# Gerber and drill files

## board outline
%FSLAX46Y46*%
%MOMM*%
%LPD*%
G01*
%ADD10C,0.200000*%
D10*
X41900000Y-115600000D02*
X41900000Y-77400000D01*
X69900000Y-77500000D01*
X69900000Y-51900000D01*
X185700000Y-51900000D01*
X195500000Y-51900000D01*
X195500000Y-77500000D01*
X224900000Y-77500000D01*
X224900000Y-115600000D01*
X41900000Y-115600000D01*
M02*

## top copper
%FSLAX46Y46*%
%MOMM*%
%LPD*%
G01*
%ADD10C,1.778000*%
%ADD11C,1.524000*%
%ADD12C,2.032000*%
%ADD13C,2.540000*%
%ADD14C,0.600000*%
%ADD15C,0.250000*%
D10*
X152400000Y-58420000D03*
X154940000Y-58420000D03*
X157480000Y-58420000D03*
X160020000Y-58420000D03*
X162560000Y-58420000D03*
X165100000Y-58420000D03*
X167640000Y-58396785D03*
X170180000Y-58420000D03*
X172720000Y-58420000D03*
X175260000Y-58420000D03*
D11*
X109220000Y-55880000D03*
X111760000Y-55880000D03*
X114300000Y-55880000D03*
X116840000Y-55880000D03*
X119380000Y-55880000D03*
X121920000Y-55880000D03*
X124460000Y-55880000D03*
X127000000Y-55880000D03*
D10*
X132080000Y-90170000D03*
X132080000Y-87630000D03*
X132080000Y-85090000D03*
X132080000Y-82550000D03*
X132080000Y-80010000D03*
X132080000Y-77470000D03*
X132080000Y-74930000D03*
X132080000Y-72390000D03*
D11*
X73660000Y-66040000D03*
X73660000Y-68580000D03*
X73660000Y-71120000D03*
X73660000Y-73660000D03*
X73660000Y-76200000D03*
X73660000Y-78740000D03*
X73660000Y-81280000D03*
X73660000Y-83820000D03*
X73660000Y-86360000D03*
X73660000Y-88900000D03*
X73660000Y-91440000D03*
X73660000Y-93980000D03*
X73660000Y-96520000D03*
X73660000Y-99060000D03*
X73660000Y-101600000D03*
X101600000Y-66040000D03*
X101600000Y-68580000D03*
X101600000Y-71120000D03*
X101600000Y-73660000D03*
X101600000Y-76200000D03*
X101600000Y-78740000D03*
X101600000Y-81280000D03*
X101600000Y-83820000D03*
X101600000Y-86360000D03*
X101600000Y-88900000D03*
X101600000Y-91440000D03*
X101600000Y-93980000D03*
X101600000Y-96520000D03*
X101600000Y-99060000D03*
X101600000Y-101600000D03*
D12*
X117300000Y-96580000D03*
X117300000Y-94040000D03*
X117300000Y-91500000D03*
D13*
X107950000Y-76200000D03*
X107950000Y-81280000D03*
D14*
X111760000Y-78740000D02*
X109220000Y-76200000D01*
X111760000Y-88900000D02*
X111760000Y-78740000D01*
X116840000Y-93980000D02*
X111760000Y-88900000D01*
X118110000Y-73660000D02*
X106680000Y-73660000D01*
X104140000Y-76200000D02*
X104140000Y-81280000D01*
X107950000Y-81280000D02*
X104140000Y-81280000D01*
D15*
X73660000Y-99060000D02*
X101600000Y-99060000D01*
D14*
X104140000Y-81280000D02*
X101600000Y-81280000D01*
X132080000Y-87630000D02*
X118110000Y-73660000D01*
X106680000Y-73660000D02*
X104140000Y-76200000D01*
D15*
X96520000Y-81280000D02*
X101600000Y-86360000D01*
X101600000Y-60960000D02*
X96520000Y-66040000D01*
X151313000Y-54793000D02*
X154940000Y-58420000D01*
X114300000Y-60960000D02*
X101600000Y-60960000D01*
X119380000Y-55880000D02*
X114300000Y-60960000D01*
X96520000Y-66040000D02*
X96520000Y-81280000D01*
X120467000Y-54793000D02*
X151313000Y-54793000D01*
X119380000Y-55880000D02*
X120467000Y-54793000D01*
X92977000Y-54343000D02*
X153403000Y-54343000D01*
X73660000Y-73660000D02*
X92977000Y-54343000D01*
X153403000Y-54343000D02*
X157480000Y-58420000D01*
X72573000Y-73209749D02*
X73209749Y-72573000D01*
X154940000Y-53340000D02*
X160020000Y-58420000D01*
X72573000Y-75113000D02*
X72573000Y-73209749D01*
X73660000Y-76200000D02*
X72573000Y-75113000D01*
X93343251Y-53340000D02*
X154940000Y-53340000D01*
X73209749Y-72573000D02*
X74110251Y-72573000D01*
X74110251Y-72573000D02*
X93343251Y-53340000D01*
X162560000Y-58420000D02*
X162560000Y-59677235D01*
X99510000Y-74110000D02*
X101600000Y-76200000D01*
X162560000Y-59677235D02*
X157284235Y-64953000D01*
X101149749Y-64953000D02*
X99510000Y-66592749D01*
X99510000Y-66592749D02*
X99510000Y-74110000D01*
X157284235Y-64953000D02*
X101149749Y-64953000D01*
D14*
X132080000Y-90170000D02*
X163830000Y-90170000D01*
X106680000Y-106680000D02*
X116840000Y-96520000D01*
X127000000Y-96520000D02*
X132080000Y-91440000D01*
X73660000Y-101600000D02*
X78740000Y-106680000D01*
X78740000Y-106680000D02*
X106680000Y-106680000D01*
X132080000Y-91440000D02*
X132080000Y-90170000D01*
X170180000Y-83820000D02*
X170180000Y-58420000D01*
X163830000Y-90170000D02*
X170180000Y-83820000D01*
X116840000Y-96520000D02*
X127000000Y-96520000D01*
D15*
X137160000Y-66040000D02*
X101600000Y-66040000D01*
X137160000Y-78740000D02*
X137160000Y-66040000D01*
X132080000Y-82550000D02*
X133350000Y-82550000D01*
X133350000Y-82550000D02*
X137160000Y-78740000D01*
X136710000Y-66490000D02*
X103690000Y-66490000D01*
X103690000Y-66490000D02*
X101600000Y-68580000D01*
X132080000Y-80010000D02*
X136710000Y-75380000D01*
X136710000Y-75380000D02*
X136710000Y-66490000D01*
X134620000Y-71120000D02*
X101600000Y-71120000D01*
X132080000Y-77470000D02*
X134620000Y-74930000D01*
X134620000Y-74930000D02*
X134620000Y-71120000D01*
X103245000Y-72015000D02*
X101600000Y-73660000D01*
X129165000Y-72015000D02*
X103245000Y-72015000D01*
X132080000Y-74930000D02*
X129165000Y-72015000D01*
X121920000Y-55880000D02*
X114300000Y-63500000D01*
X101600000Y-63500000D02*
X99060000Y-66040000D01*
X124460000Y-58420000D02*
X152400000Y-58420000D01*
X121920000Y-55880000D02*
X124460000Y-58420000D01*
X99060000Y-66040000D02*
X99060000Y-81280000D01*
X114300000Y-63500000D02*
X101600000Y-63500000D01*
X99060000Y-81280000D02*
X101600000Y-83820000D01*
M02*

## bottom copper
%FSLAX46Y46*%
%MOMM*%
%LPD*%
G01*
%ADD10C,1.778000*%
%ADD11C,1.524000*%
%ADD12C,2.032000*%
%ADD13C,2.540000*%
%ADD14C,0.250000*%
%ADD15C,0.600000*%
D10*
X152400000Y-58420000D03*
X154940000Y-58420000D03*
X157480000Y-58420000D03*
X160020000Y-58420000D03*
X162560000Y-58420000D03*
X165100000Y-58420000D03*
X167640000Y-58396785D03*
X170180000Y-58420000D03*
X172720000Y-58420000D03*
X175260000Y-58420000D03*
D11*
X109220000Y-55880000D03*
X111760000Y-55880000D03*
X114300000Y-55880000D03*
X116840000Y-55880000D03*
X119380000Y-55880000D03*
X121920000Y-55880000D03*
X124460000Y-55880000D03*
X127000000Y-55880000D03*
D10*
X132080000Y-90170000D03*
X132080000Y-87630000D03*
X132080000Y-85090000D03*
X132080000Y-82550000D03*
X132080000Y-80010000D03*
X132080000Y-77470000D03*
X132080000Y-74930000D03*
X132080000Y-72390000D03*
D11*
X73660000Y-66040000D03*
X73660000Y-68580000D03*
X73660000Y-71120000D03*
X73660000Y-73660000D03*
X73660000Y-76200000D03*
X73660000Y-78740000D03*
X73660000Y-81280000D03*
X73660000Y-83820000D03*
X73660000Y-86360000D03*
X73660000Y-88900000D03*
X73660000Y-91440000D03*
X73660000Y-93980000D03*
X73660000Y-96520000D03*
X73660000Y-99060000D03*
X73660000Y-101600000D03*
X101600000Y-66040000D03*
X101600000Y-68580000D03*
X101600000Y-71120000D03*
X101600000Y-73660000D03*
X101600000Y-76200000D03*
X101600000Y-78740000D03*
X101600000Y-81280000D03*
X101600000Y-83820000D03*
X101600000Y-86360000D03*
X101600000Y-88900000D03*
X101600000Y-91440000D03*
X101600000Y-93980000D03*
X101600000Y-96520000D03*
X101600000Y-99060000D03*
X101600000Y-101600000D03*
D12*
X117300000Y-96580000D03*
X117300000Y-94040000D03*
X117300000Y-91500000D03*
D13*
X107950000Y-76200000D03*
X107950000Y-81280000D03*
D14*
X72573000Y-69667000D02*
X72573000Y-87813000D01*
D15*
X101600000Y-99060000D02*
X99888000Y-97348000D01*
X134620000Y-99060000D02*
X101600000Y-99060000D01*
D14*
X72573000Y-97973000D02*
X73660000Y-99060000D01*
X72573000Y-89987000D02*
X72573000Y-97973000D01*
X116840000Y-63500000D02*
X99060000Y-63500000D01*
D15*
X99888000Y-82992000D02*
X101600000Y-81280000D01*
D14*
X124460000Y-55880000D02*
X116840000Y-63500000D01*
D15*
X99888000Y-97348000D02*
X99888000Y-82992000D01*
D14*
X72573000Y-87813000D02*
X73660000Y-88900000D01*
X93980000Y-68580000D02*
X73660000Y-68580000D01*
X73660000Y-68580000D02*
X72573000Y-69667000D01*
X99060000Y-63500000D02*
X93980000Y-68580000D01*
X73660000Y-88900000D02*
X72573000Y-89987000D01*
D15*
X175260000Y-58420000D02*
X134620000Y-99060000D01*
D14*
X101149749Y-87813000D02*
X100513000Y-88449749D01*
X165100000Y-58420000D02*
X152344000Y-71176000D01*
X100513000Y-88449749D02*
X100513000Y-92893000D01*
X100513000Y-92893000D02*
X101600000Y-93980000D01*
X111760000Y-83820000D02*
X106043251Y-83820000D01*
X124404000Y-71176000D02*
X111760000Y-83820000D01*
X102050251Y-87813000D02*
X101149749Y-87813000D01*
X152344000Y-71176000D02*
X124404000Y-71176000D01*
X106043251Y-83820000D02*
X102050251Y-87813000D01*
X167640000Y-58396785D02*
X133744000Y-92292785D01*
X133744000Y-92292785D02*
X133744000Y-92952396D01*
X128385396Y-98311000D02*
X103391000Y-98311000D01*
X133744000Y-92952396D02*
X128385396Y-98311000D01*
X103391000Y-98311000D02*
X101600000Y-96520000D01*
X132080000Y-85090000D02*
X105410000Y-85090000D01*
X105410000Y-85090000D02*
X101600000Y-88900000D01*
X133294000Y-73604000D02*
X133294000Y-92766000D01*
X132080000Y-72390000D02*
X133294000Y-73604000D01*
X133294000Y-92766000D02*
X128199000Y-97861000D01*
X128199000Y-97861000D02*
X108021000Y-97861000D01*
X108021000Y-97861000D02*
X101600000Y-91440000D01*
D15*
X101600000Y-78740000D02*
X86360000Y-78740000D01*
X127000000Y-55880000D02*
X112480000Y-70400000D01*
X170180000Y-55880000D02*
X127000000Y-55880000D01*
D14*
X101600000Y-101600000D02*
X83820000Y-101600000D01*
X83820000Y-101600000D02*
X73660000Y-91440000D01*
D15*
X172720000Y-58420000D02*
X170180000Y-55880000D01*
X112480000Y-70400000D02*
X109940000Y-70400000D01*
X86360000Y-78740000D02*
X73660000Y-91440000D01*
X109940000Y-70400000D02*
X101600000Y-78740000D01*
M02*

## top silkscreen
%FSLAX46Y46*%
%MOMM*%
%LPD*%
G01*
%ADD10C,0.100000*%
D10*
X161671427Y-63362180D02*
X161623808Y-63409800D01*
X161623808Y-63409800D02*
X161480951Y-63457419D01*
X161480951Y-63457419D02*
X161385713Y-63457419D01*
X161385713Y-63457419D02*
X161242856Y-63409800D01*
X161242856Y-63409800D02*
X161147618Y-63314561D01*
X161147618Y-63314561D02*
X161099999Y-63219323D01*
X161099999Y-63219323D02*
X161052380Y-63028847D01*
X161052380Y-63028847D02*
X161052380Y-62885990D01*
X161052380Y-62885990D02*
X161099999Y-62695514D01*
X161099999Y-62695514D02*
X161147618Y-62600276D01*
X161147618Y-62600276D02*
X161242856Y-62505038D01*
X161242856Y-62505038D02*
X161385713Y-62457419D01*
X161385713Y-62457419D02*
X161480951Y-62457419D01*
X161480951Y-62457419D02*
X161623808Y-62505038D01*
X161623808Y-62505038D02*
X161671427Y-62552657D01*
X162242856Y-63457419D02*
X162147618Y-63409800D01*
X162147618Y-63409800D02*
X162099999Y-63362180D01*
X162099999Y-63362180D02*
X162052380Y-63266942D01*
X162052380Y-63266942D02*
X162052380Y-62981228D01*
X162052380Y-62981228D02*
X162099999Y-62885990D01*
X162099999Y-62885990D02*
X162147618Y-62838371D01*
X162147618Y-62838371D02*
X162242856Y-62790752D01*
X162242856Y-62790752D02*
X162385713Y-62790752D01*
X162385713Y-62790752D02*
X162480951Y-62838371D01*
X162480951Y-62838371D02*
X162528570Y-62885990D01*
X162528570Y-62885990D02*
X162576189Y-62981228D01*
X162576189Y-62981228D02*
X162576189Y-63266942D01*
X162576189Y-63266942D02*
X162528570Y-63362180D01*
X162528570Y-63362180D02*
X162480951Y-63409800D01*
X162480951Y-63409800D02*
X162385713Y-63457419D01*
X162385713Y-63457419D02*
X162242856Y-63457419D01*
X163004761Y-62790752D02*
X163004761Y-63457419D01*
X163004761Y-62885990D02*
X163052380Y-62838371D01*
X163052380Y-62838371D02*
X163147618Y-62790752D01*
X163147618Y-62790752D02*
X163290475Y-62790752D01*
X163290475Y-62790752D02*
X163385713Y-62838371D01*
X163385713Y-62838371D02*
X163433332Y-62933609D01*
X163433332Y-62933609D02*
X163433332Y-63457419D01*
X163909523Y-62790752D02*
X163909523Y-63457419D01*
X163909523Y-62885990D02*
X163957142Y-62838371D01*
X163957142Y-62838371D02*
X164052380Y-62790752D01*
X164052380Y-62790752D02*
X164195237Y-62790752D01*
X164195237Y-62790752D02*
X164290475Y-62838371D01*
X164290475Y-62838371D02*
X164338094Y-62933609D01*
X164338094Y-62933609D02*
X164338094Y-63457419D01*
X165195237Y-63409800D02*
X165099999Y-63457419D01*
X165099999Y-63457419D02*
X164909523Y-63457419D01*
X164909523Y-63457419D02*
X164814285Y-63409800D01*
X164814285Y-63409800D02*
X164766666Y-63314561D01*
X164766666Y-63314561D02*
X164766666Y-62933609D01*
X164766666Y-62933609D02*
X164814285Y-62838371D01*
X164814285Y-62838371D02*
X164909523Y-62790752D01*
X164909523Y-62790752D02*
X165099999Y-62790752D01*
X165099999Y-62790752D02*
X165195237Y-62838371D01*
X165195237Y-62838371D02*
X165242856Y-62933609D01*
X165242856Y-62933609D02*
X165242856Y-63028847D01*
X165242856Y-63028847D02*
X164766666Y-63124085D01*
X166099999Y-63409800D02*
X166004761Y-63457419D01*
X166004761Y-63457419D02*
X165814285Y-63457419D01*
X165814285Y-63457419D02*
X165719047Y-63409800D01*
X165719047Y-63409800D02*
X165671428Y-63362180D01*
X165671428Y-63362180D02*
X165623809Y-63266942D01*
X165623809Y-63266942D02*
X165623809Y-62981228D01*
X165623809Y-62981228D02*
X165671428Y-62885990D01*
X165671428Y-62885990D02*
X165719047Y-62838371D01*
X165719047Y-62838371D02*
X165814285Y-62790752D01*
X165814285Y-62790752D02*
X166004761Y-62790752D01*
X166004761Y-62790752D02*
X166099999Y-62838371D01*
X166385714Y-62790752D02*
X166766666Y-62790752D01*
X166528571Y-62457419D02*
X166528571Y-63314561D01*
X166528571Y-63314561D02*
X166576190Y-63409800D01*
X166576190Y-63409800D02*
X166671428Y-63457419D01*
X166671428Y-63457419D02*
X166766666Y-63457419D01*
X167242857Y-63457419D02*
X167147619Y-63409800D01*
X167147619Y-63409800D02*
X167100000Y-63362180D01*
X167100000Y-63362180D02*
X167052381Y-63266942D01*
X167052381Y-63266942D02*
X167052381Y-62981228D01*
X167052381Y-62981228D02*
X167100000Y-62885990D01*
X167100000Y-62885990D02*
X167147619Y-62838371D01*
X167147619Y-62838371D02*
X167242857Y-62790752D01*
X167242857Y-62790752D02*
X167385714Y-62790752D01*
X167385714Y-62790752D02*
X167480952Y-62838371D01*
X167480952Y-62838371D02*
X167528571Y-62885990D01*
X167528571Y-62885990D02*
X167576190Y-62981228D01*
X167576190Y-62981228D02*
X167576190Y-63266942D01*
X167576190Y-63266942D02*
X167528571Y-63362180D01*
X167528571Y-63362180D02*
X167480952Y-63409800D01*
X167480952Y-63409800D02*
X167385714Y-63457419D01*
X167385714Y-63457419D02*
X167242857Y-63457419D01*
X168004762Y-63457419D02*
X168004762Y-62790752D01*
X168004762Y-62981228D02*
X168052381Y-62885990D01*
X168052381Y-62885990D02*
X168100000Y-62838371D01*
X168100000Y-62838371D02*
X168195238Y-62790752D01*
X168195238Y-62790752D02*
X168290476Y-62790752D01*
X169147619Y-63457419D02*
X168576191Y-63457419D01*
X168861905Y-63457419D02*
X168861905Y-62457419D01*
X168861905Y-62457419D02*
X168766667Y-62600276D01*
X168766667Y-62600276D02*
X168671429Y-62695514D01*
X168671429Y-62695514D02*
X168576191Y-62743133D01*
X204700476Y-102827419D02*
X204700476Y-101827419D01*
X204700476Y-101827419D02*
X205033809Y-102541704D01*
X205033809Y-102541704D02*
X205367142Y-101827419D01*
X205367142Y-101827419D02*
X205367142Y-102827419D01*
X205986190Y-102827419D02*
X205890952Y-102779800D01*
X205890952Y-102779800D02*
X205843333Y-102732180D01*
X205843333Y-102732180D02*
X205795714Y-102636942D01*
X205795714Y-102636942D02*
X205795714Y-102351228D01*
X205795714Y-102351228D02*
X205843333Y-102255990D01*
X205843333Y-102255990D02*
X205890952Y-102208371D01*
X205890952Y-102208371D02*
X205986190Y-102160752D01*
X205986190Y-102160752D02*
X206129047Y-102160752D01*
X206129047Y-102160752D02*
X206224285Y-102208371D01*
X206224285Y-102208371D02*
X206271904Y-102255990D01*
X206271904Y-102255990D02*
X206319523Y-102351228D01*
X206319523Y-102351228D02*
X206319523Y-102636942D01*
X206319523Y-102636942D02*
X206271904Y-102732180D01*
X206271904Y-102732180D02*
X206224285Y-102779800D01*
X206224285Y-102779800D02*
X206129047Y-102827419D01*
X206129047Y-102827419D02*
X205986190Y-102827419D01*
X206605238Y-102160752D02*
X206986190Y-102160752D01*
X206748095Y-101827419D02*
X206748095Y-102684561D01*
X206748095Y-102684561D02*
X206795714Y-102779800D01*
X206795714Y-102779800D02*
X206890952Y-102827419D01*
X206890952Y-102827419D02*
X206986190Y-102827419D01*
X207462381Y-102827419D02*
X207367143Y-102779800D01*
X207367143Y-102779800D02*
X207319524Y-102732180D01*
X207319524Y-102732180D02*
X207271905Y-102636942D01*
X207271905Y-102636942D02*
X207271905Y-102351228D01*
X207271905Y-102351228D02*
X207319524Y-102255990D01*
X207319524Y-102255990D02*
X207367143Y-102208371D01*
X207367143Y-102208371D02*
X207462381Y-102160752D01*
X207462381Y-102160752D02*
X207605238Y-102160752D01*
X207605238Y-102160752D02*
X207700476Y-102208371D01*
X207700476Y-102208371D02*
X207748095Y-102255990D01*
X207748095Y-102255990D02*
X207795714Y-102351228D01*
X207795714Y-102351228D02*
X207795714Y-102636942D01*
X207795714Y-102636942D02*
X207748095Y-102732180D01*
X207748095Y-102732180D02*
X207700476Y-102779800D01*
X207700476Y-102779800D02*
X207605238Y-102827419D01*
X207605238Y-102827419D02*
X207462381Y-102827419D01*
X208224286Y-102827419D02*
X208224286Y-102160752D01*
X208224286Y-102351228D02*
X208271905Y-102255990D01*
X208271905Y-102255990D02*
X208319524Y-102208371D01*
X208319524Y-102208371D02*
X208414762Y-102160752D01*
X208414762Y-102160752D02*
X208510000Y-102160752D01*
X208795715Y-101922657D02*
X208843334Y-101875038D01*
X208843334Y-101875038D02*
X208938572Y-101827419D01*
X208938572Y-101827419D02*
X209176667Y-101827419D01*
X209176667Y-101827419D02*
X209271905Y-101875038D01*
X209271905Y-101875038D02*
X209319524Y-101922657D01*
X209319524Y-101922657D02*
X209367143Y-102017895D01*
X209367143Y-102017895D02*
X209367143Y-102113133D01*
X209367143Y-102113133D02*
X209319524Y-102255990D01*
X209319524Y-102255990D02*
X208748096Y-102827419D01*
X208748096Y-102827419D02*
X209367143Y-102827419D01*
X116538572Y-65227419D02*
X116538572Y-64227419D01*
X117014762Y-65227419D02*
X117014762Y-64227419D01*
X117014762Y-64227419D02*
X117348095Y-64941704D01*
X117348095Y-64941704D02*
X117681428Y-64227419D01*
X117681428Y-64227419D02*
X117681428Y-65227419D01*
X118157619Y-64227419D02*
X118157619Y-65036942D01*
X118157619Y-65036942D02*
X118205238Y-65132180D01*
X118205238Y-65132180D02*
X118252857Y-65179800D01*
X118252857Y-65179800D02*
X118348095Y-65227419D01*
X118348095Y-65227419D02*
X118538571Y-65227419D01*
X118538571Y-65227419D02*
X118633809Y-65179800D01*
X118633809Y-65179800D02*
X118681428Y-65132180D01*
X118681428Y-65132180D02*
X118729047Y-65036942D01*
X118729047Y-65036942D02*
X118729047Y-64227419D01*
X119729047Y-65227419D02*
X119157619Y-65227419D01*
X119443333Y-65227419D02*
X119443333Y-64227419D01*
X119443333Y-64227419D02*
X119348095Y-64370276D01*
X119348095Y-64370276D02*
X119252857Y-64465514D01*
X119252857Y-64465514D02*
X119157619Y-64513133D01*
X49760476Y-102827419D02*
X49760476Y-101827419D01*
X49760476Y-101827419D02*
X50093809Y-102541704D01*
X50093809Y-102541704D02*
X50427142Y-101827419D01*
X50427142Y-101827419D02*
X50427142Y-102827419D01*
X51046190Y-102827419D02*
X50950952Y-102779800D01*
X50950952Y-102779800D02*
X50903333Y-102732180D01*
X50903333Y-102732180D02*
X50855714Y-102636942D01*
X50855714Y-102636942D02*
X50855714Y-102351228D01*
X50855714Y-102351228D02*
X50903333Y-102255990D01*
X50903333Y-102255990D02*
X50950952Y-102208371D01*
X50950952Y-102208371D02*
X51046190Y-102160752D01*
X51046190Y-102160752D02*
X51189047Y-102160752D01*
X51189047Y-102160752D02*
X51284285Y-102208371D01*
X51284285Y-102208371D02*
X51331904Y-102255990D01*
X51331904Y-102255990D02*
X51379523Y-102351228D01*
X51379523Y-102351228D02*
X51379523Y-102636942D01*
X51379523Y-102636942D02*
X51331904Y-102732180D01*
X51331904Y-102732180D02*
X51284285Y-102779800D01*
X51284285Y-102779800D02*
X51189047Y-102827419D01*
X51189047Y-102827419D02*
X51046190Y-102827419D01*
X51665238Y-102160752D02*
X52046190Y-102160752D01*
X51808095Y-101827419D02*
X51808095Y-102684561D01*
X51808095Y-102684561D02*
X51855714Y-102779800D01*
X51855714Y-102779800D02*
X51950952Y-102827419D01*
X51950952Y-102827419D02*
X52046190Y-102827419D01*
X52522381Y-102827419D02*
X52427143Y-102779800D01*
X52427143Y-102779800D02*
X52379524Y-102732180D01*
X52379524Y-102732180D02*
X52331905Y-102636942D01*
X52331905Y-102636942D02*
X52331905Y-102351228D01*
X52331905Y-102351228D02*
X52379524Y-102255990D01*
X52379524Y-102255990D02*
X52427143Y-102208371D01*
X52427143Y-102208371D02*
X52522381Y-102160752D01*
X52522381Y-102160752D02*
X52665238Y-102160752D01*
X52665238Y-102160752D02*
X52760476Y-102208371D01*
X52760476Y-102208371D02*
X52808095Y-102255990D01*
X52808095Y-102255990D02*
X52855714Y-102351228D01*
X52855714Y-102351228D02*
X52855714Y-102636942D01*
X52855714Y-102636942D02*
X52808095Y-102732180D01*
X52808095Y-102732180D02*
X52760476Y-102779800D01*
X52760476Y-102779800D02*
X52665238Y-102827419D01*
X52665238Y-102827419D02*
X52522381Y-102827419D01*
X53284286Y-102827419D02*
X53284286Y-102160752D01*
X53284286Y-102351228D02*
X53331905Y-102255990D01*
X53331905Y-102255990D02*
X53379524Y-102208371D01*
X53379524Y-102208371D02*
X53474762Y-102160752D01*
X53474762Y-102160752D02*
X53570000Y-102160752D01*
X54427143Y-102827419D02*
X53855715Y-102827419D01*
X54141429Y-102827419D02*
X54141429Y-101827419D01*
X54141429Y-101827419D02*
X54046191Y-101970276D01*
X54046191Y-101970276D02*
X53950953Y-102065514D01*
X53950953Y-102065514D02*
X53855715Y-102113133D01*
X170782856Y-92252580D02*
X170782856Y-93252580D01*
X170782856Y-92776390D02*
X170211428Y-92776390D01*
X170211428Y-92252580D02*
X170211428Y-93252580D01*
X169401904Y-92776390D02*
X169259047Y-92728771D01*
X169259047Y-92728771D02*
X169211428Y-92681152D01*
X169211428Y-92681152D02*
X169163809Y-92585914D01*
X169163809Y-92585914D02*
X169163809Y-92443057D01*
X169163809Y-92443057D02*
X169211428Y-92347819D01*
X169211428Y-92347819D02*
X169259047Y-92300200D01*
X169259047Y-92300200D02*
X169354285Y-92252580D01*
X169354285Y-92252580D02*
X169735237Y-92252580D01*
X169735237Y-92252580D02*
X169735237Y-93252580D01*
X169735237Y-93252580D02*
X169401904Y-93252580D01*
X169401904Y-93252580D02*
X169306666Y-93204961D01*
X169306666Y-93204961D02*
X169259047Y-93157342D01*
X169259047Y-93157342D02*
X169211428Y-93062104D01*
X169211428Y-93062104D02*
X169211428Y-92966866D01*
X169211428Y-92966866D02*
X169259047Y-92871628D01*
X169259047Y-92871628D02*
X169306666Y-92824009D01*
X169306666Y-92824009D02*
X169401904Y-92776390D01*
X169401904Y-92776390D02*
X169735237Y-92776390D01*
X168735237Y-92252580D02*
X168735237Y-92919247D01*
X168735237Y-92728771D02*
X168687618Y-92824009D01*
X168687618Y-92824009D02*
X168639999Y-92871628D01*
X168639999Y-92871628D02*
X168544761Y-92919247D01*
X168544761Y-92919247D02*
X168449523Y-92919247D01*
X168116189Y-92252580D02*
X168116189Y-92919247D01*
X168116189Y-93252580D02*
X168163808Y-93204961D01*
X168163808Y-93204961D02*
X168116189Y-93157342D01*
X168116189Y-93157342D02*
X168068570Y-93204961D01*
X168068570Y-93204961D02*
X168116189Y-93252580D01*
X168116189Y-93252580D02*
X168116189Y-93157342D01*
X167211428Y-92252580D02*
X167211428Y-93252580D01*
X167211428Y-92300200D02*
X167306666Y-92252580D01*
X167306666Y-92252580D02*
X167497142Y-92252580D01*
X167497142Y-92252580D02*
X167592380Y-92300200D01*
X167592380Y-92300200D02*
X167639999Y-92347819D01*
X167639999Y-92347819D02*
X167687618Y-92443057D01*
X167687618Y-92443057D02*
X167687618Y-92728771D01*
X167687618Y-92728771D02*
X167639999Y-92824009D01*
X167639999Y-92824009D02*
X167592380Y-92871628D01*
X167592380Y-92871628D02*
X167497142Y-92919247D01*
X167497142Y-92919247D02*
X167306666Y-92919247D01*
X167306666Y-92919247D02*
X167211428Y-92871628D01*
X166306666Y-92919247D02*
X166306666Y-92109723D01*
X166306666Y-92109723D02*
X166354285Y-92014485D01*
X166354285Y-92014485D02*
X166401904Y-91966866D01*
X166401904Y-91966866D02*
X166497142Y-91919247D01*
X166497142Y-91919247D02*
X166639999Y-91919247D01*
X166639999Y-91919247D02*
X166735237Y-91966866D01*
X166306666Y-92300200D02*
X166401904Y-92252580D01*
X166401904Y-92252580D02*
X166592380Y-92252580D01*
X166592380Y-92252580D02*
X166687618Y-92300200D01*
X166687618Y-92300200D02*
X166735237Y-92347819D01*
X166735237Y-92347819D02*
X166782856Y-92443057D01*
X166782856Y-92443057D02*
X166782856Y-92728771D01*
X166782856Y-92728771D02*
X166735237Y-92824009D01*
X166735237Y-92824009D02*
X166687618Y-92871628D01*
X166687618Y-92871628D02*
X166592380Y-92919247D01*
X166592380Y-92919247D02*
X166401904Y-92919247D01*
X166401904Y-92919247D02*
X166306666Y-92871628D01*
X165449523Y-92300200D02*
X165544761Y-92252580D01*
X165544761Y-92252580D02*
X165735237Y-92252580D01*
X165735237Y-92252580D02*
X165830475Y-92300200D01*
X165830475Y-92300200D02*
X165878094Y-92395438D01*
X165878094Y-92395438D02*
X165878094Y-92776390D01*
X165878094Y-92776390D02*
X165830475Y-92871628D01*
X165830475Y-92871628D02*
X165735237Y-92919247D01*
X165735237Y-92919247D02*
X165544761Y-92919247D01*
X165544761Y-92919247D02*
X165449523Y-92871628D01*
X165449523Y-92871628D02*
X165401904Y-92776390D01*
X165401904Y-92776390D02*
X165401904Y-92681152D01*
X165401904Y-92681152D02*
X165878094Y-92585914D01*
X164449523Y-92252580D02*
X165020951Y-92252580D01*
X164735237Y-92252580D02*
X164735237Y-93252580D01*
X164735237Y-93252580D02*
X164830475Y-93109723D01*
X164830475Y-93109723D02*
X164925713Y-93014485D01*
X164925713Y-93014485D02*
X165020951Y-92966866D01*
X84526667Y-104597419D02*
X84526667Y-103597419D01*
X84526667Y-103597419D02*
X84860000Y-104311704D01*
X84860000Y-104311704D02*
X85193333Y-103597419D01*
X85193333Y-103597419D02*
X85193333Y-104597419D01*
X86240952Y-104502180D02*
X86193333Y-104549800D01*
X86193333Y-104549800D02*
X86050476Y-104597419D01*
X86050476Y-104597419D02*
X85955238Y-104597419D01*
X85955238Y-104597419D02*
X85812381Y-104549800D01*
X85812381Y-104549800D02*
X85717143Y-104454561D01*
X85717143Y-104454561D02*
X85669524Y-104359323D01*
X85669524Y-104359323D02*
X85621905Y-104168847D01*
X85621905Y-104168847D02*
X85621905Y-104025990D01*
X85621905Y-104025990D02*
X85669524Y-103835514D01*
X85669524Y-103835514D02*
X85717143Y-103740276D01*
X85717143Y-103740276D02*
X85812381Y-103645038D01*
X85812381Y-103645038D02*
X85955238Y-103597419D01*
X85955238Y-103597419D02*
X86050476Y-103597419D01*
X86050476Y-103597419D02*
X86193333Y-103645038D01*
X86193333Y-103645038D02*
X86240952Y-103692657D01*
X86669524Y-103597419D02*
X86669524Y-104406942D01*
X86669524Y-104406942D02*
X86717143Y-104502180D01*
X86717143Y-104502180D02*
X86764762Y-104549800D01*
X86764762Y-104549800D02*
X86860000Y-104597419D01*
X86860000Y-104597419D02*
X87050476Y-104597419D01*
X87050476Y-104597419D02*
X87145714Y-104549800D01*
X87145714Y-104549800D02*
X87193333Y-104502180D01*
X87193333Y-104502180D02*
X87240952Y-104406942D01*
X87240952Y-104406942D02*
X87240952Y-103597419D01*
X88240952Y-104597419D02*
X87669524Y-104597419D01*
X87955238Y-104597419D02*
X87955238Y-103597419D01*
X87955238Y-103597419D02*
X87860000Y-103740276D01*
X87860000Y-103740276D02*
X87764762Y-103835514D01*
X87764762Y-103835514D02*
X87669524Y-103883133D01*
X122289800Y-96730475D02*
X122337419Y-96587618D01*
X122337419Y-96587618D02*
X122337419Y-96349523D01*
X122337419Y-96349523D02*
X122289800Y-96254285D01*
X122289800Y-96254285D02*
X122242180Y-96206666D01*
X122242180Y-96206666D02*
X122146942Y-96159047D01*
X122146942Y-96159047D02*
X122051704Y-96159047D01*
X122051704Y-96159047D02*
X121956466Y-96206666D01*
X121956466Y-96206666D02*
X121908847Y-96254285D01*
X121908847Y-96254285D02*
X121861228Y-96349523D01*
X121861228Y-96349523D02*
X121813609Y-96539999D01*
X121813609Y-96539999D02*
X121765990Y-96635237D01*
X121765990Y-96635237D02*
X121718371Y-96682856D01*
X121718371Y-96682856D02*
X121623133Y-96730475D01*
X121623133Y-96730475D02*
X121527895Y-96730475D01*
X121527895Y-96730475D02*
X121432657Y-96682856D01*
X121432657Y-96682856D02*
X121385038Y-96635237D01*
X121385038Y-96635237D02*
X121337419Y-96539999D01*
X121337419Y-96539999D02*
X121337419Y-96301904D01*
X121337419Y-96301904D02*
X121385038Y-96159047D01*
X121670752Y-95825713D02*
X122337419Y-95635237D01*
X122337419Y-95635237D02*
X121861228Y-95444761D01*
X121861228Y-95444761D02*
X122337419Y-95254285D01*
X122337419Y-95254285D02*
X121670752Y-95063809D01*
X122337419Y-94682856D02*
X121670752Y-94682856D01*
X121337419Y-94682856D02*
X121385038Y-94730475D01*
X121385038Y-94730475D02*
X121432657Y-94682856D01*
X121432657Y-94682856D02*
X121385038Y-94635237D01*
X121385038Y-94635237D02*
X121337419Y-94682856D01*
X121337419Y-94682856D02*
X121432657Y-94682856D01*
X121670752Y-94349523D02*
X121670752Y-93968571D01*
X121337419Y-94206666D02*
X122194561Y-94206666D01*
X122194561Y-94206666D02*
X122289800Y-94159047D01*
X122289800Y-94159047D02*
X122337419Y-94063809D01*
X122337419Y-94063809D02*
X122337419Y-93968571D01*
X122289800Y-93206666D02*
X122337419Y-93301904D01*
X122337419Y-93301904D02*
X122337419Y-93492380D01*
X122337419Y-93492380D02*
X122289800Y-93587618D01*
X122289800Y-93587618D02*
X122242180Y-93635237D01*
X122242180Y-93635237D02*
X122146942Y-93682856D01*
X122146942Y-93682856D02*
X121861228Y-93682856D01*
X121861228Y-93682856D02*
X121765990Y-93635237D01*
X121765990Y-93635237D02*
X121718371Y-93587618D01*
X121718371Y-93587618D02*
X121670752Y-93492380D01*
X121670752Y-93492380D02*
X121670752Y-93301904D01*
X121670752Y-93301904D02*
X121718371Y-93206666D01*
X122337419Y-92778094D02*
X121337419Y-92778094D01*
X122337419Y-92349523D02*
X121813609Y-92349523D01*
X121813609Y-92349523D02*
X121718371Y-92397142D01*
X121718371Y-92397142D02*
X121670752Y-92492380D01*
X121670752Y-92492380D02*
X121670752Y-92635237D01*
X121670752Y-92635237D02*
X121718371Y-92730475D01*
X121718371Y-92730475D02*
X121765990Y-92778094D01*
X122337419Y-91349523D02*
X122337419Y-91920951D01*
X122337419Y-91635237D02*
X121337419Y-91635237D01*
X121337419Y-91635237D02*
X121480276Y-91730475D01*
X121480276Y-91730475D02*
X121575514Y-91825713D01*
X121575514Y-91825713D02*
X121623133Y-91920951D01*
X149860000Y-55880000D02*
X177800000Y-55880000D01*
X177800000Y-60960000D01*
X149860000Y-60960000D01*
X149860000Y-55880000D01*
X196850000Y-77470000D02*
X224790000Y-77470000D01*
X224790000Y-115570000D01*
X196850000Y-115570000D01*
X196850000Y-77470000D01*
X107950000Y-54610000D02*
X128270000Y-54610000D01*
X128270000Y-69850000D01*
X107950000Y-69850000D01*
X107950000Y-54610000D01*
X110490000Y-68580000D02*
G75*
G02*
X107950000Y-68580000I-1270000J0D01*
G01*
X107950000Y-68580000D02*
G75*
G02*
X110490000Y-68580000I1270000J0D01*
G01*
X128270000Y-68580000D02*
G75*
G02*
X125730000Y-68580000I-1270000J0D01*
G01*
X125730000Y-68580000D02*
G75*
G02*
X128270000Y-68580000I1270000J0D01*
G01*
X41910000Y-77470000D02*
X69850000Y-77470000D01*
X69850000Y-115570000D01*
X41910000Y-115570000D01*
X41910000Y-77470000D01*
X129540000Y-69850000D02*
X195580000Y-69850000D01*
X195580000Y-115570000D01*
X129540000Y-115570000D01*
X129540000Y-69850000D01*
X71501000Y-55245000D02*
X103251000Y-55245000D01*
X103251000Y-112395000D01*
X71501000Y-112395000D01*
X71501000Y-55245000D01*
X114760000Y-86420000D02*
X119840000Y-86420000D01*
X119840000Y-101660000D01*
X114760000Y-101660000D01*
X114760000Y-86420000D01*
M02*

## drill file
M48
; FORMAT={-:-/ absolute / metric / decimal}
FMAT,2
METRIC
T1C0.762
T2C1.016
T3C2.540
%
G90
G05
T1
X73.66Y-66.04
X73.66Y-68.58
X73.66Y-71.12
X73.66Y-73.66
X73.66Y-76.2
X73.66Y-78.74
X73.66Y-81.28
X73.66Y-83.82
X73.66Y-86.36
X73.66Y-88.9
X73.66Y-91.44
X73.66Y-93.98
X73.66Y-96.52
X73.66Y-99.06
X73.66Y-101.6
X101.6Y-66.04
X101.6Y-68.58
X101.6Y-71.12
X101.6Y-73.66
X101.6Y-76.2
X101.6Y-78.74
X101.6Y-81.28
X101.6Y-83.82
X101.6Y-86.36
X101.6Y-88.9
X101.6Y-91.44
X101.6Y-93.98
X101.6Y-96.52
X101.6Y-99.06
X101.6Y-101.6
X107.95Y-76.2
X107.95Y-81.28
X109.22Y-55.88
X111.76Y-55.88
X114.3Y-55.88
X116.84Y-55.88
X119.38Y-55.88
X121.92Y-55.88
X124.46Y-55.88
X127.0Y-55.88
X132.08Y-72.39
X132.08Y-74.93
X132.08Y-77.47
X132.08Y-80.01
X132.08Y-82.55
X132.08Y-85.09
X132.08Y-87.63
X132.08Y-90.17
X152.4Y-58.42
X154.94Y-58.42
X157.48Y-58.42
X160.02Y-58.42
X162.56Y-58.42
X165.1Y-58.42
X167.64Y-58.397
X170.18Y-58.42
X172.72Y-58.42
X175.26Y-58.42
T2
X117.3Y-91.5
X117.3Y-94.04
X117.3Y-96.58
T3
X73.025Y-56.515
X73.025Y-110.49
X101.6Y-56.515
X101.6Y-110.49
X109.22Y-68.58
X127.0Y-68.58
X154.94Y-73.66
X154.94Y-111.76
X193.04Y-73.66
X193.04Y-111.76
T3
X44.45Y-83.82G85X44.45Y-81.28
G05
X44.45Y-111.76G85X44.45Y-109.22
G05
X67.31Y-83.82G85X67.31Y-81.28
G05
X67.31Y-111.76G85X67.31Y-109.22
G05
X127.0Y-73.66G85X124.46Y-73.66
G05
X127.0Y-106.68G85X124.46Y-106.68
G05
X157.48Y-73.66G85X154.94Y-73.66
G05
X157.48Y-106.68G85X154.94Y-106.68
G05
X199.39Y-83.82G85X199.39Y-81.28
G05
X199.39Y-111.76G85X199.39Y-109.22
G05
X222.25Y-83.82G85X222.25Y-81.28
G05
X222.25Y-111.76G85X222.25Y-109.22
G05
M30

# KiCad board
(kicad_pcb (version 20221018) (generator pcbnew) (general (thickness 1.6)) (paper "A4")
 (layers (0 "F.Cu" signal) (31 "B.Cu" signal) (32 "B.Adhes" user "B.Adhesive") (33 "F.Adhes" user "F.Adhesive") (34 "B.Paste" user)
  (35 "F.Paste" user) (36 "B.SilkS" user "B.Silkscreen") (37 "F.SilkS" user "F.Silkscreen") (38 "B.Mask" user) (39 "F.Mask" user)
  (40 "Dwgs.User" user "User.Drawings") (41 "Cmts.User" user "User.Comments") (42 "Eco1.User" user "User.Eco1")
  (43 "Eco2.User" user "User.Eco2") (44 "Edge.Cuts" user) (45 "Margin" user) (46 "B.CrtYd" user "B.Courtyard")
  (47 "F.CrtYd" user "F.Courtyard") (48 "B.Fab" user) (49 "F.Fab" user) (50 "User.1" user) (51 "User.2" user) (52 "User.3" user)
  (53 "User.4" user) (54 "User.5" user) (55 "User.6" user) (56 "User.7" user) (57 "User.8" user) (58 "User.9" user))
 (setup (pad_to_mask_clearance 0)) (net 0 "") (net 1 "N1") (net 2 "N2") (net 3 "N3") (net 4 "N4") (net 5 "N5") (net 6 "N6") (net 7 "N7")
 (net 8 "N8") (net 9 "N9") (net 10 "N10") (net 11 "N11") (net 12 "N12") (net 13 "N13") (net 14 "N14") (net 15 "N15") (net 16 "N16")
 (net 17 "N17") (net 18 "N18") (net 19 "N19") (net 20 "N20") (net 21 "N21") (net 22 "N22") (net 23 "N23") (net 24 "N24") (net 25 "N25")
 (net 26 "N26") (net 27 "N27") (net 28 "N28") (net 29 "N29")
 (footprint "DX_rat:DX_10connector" (layer "F.Cu") (at 165.1 63.5)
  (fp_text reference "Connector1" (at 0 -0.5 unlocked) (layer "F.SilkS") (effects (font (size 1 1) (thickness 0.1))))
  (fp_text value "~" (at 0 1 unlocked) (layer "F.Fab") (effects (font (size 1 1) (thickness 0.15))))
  (fp_rect (start -15.24 -7.62) (end 12.7 -2.54) (stroke (width 0.1) (type default)) (fill none) (layer "F.SilkS"))
  (pad "1" thru_hole circle (at -12.7 -5.08) (size 1.778 1.778) (drill 0.762) (layers "*.Cu" "*.Mask") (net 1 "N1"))
  (pad "2" thru_hole circle (at -10.16 -5.08) (size 1.778 1.778) (drill 0.762) (layers "*.Cu" "*.Mask") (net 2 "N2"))
  (pad "3" thru_hole circle (at -7.62 -5.08) (size 1.778 1.778) (drill 0.762) (layers "*.Cu" "*.Mask") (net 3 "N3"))
  (pad "4" thru_hole circle (at -5.08 -5.08) (size 1.778 1.778) (drill 0.762) (layers "*.Cu" "*.Mask") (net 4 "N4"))
  (pad "5" thru_hole circle (at -2.54 -5.08) (size 1.778 1.778) (drill 0.762) (layers "*.Cu" "*.Mask") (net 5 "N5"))
  (pad "6" thru_hole circle (at 0 -5.08) (size 1.778 1.778) (drill 0.762) (layers "*.Cu" "*.Mask") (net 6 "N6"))
  (pad "7" thru_hole circle (at 2.54 -5.103215) (size 1.778 1.778) (drill 0.762) (layers "*.Cu" "*.Mask") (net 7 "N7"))
  (pad "8" thru_hole circle (at 5.08 -5.08) (size 1.778 1.778) (drill 0.762) (layers "*.Cu" "*.Mask") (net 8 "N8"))
  (pad "9" thru_hole circle (at 7.62 -5.08) (size 1.778 1.778) (drill 0.762) (layers "*.Cu" "*.Mask") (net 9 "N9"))
  (pad "10" thru_hole circle (at 10.16 -5.08) (size 1.778 1.778) (drill 0.762) (layers "*.Cu" "*.Mask" "Dwgs.User") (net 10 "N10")))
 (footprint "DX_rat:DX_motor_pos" (layer "F.Cu") (at 207.01 102.87)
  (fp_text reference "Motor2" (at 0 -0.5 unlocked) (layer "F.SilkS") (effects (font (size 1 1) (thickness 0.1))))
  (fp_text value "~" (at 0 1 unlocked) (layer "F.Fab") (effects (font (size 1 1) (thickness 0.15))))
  (fp_rect (start -10.16 -25.4) (end 17.78 12.7) (stroke (width 0.1) (type default)) (fill none) (layer "F.SilkS"))
  (pad "" np_thru_hole oval (at -7.62 -20.32 90) (size 5.08 2.54) (drill oval 5.08 2.54) (layers "F&B.Cu" "*.Mask"))
  (pad "" np_thru_hole oval (at -7.62 7.62 90) (size 5.08 2.54) (drill oval 5.08 2.54) (layers "F&B.Cu" "*.Mask"))
  (pad "" np_thru_hole oval (at 15.24 -20.32 90) (size 5.08 2.54) (drill oval 5.08 2.54) (layers "F&B.Cu" "*.Mask"))
  (pad "" np_thru_hole oval (at 15.24 7.62 90) (size 5.08 2.54) (drill oval 5.08 2.54) (layers "F&B.Cu" "*.Mask")))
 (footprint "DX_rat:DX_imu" (layer "F.Cu") (at 116.84 60.96)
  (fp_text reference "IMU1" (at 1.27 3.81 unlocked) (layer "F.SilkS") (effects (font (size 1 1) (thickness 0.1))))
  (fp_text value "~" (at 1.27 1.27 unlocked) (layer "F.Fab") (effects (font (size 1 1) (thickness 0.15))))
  (fp_rect (start -8.89 -6.35) (end 11.43 8.89) (stroke (width 0.1) (type default)) (fill none) (layer "F.SilkS"))
  (fp_circle (center -7.62 7.62) (end -7.62 8.89) (stroke (width 0.1) (type default)) (fill none) (layer "F.SilkS"))
  (fp_circle (center 10.16 7.62) (end 11.43 7.62) (stroke (width 0.1) (type default)) (fill none) (layer "F.SilkS"))
  (pad "" np_thru_hole circle (at -7.62 7.62) (size 2.54 2.54) (drill 2.54) (layers "F&B.Cu" "*.Mask"))
  (pad "" np_thru_hole circle (at 10.16 7.62) (size 2.54 2.54) (drill 2.54) (layers "F&B.Cu" "*.Mask"))
  (pad "1" thru_hole circle (at -7.62 -5.08) (size 1.524 1.524) (drill 0.762) (layers "*.Cu" "*.Mask") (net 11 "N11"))
  (pad "2" thru_hole circle (at -5.08 -5.08) (size 1.524 1.524) (drill 0.762) (layers "*.Cu" "*.Mask") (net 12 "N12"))
  (pad "3" thru_hole circle (at -2.54 -5.08) (size 1.524 1.524) (drill 0.762) (layers "*.Cu" "*.Mask") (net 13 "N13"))
  (pad "4" thru_hole circle (at 0 -5.08) (size 1.524 1.524) (drill 0.762) (layers "*.Cu" "*.Mask") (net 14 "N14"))
  (pad "5" thru_hole circle (at 2.54 -5.08) (size 1.524 1.524) (drill 0.762) (layers "*.Cu" "*.Mask") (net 2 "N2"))
  (pad "6" thru_hole circle (at 5.08 -5.08) (size 1.524 1.524) (drill 0.762) (layers "*.Cu" "*.Mask") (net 1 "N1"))
  (pad "7" thru_hole circle (at 7.62 -5.08) (size 1.524 1.524) (drill 0.762) (layers "*.Cu" "*.Mask") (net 10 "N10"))
  (pad "8" thru_hole circle (at 10.16 -5.08) (size 1.524 1.524) (drill 0.762) (layers "*.Cu" "*.Mask") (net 9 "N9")))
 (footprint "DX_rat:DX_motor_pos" (layer "F.Cu") (at 52.07 102.87)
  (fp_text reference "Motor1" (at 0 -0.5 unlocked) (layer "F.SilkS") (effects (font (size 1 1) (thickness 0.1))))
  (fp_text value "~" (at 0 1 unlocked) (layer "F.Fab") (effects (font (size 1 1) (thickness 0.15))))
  (fp_rect (start -10.16 -25.4) (end 17.78 12.7) (stroke (width 0.1) (type default)) (fill none) (layer "F.SilkS"))
  (pad "" np_thru_hole oval (at -7.62 -20.32 90) (size 5.08 2.54) (drill oval 5.08 2.54) (layers "F&B.Cu" "*.Mask"))
  (pad "" np_thru_hole oval (at -7.62 7.62 90) (size 5.08 2.54) (drill oval 5.08 2.54) (layers "F&B.Cu" "*.Mask"))
  (pad "" np_thru_hole oval (at 15.24 -20.32 90) (size 5.08 2.54) (drill oval 5.08 2.54) (layers "F&B.Cu" "*.Mask"))
  (pad "" np_thru_hole oval (at 15.24 7.62 90) (size 5.08 2.54) (drill oval 5.08 2.54) (layers "F&B.Cu" "*.Mask")))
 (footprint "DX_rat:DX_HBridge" (layer "F.Cu") (at 170.18 102.87 180)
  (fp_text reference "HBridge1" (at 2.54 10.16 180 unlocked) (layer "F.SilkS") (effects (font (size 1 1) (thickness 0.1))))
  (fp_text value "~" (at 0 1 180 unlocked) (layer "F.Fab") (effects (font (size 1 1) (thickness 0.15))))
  (fp_rect (start -25.4 -12.7) (end 40.64 33.02) (stroke (width 0.1) (type default)) (fill none) (layer "F.SilkS"))
  (pad "" np_thru_hole circle (at -22.86 -8.89 180) (size 2.54 2.54) (drill 2.54) (layers "F&B.Cu" "*.Mask"))
  (pad "" np_thru_hole circle (at -22.86 29.21 180) (size 2.54 2.54) (drill 2.54) (layers "F&B.Cu" "*.Mask"))
  (pad "" np_thru_hole circle (at 15.24 -8.89 180) (size 2.54 2.54) (drill 2.54) (layers "F&B.Cu" "*.Mask"))
  (pad "" np_thru_hole circle (at 15.24 29.21 180) (size 2.54 2.54) (drill 2.54) (layers "F&B.Cu" "*.Mask"))
  (pad "1" thru_hole circle (at 38.1 12.7 180) (size 1.778 1.778) (drill 0.762) (layers "*.Cu" "*.Mask") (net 8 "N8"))
  (pad "2" thru_hole circle (at 38.1 15.24 180) (size 1.778 1.778) (drill 0.762) (layers "*.Cu" "*.Mask") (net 10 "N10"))
  (pad "3" thru_hole circle (at 38.1 17.78 180) (size 1.778 1.778) (drill 0.762) (layers "*.Cu" "*.Mask") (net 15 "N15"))
  (pad "4" thru_hole circle (at 38.1 20.32 180) (size 1.778 1.778) (drill 0.762) (layers "*.Cu" "*.Mask") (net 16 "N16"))
  (pad "5" thru_hole circle (at 38.1 22.86 180) (size 1.778 1.778) (drill 0.762) (layers "*.Cu" "*.Mask") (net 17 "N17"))
  (pad "6" thru_hole circle (at 38.1 25.4 180) (size 1.778 1.778) (drill 0.762) (layers "*.Cu" "*.Mask") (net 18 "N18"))
  (pad "7" thru_hole circle (at 38.1 27.94 180) (size 1.778 1.778) (drill 0.762) (layers "*.Cu" "*.Mask") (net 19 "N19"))
  (pad "8" thru_hole circle (at 38.1 30.48 180) (size 1.778 1.778) (drill 0.762) (layers "*.Cu" "*.Mask") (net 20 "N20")))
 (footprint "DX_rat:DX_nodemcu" (layer "F.Cu") (at 81.28 91.44)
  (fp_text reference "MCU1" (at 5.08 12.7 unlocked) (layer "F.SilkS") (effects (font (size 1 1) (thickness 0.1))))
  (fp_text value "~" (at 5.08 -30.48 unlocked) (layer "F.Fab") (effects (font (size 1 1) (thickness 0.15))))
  (fp_rect (start -9.779 -36.195) (end 21.971 20.955) (stroke (width 0.1) (type default)) (fill none) (layer "F.SilkS"))
  (pad "" np_thru_hole circle (at -8.255 -34.925) (size 2.54 2.54) (drill 2.54) (layers "F&B.Cu" "*.Mask"))
  (pad "" np_thru_hole circle (at -8.255 19.05) (size 2.54 2.54) (drill 2.54) (layers "F&B.Cu" "*.Mask"))
  (pad "" np_thru_hole circle (at 20.32 -34.925) (size 2.54 2.54) (drill 2.54) (layers "F&B.Cu" "*.Mask"))
  (pad "" np_thru_hole circle (at 20.32 19.05) (size 2.54 2.54) (drill 2.54) (layers "F&B.Cu" "*.Mask"))
  (pad "1" thru_hole circle (at -7.62 -25.4) (size 1.524 1.524) (drill 0.762) (layers "*.Cu" "*.Mask") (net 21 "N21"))
  (pad "2" thru_hole circle (at -7.62 -22.86) (size 1.524 1.524) (drill 0.762) (layers "*.Cu" "*.Mask") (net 10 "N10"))
  (pad "3" thru_hole circle (at -7.62 -20.32) (size 1.524 1.524) (drill 0.762) (layers "*.Cu" "*.Mask"))
  (pad "4" thru_hole circle (at -7.62 -17.78) (size 1.524 1.524) (drill 0.762) (layers "*.Cu" "*.Mask") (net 3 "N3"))
  (pad "5" thru_hole circle (at -7.62 -15.24) (size 1.524 1.524) (drill 0.762) (layers "*.Cu" "*.Mask") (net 4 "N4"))
  (pad "6" thru_hole circle (at -7.62 -12.7) (size 1.524 1.524) (drill 0.762) (layers "*.Cu" "*.Mask") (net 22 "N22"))
  (pad "7" thru_hole circle (at -7.62 -10.16) (size 1.524 1.524) (drill 0.762) (layers "*.Cu" "*.Mask") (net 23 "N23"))
  (pad "8" thru_hole circle (at -7.62 -7.62) (size 1.524 1.524) (drill 0.762) (layers "*.Cu" "*.Mask") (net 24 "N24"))
  (pad "9" thru_hole circle (at -7.62 -5.08) (size 1.524 1.524) (drill 0.762) (layers "*.Cu" "*.Mask") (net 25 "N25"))
  (pad "10" thru_hole circle (at -7.62 -2.54) (size 1.524 1.524) (drill 0.762) (layers "*.Cu" "*.Mask") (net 10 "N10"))
  (pad "11" thru_hole circle (at -7.62 0) (size 1.524 1.524) (drill 0.762) (layers "*.Cu" "*.Mask") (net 9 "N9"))
  (pad "12" thru_hole circle (at -7.62 2.54) (size 1.524 1.524) (drill 0.762) (layers "*.Cu" "*.Mask") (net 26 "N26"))
  (pad "13" thru_hole circle (at -7.62 5.08) (size 1.524 1.524) (drill 0.762) (layers "*.Cu" "*.Mask") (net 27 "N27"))
  (pad "14" thru_hole circle (at -7.62 7.62) (size 1.524 1.524) (drill 0.762) (layers "*.Cu" "*.Mask") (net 10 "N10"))
  (pad "15" thru_hole circle (at -7.62 10.16) (size 1.524 1.524) (drill 0.762) (layers "*.Cu" "*.Mask") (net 8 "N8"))
  (pad "16" thru_hole circle (at 20.32 -25.4) (size 1.524 1.524) (drill 0.762) (layers "*.Cu" "*.Mask") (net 16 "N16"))
  (pad "17" thru_hole circle (at 20.32 -22.86) (size 1.524 1.524) (drill 0.762) (layers "*.Cu" "*.Mask") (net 17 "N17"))
  (pad "18" thru_hole circle (at 20.32 -20.32) (size 1.524 1.524) (drill 0.762) (layers "*.Cu" "*.Mask") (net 18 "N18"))
  (pad "19" thru_hole circle (at 20.32 -17.78) (size 1.524 1.524) (drill 0.762) (layers "*.Cu" "*.Mask") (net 19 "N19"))
  (pad "20" thru_hole circle (at 20.32 -15.24) (size 1.524 1.524) (drill 0.762) (layers "*.Cu" "*.Mask") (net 5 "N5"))
  (pad "21" thru_hole circle (at 20.32 -12.7) (size 1.524 1.524) (drill 0.762) (layers "*.Cu" "*.Mask") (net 9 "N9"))
  (pad "22" thru_hole circle (at 20.32 -10.16) (size 1.524 1.524) (drill 0.762) (layers "*.Cu" "*.Mask") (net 10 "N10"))
  (pad "23" thru_hole circle (at 20.32 -7.62) (size 1.524 1.524) (drill 0.762) (layers "*.Cu" "*.Mask") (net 1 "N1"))
  (pad "24" thru_hole circle (at 20.32 -5.08) (size 1.524 1.524) (drill 0.762) (layers "*.Cu" "*.Mask") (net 2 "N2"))
  (pad "25" thru_hole circle (at 20.32 -2.54) (size 1.524 1.524) (drill 0.762) (layers "*.Cu" "*.Mask") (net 15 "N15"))
  (pad "26" thru_hole circle (at 20.32 0) (size 1.524 1.524) (drill 0.762) (layers "*.Cu" "*.Mask") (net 20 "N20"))
  (pad "27" thru_hole circle (at 20.32 2.54) (size 1.524 1.524) (drill 0.762) (layers "*.Cu" "*.Mask") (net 6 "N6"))
  (pad "28" thru_hole circle (at 20.32 5.08) (size 1.524 1.524) (drill 0.762) (layers "*.Cu" "*.Mask") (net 7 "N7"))
  (pad "29" thru_hole circle (at 20.32 7.62) (size 1.524 1.524) (drill 0.762) (layers "*.Cu" "*.Mask") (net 10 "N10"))
  (pad "30" thru_hole circle (at 20.32 10.16) (size 1.524 1.524) (drill 0.762) (layers "*.Cu" "*.Mask") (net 9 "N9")))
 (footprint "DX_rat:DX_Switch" (layer "F.Cu") (at 122.38 94.04 90)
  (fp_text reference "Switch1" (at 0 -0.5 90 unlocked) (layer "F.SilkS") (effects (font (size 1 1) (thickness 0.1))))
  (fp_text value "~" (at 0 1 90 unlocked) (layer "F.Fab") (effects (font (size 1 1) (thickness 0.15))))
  (fp_rect (start -7.62 -2.54) (end 7.62 -7.62) (stroke (width 0.1) (type default)) (fill none) (layer "F.SilkS"))
  (pad "1" thru_hole circle (at -2.54 -5.08 90) (size 2.032 2.032) (drill 1.016) (layers "*.Cu" "*.Mask") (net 8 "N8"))
  (pad "2" thru_hole circle (at 0 -5.08 90) (size 2.032 2.032) (drill 1.016) (layers "*.Cu" "*.Mask") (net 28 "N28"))
  (pad "3" thru_hole circle (at 2.54 -5.08 90) (size 2.032 2.032) (drill 1.016) (layers "*.Cu" "*.Mask") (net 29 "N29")))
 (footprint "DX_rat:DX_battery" (layer "B.Cu") (at 156.21 81.28 180)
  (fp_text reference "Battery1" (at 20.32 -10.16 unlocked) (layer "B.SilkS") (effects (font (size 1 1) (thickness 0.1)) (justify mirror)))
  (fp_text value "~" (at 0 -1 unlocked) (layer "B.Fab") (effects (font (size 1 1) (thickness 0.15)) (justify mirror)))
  (pad "" np_thru_hole oval (at 0 -25.4 180) (size 5.08 2.54) (drill oval 5.08 2.54) (layers "F&B.Cu" "*.Mask"))
  (pad "" np_thru_hole oval (at 0 7.62 180) (size 5.08 2.54) (drill oval 5.08 2.54) (layers "F&B.Cu" "*.Mask"))
  (pad "" np_thru_hole oval (at 30.48 -25.4 180) (size 5.08 2.54) (drill oval 5.08 2.54) (layers "F&B.Cu" "*.Mask"))
  (pad "" np_thru_hole oval (at 30.48 7.62 180) (size 5.08 2.54) (drill oval 5.08 2.54) (layers "F&B.Cu" "*.Mask"))
  (pad "1" thru_hole circle (at 48.26 5.08 180) (size 2.54 2.54) (drill 0.762) (layers "*.Cu" "*.Mask") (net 28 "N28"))
  (pad "2" thru_hole circle (at 48.26 0 180) (size 2.54 2.54) (drill 0.762) (layers "*.Cu" "*.Mask") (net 10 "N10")))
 (gr_poly
  (pts (xy 41.9 115.6) (xy 41.9 77.4) (xy 69.9 77.5) (xy 69.9 51.9) (xy 185.7 51.9) (xy 195.5 51.9) (xy 195.5 77.5) (xy 224.9 77.5)
   (xy 224.9 115.6))
  (stroke (width 0.2) (type solid)) (fill none) (layer "Edge.Cuts"))
 (segment (start 111.76 78.74) (end 109.22 76.2) (width 0.6) (layer "F.Cu") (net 28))
 (segment (start 111.76 88.9) (end 111.76 78.74) (width 0.6) (layer "F.Cu") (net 28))
 (segment (start 116.84 93.98) (end 111.76 88.9) (width 0.6) (layer "F.Cu") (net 28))
 (segment (start 118.11 73.66) (end 106.68 73.66) (width 0.6) (layer "F.Cu") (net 10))
 (segment (start 104.14 76.2) (end 104.14 81.28) (width 0.6) (layer "F.Cu") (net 10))
 (segment (start 107.95 81.28) (end 104.14 81.28) (width 0.6) (layer "F.Cu") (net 10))
 (segment (start 73.66 99.06) (end 101.6 99.06) (width 0.25) (layer "F.Cu") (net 10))
 (segment (start 104.14 81.28) (end 101.6 81.28) (width 0.6) (layer "F.Cu") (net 10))
 (segment (start 132.08 87.63) (end 118.11 73.66) (width 0.6) (layer "F.Cu") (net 10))
 (segment (start 106.68 73.66) (end 104.14 76.2) (width 0.6) (layer "F.Cu") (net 10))
 (segment (start 72.573 69.667) (end 72.573 87.813) (width 0.25) (layer "B.Cu") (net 10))
 (segment (start 101.6 99.06) (end 99.888 97.348) (width 0.6) (layer "B.Cu") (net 10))
 (segment (start 134.62 99.06) (end 101.6 99.06) (width 0.6) (layer "B.Cu") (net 10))
 (segment (start 72.573 97.973) (end 73.66 99.06) (width 0.25) (layer "B.Cu") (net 10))
 (segment (start 72.573 89.987) (end 72.573 97.973) (width 0.25) (layer "B.Cu") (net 10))
 (segment (start 116.84 63.5) (end 99.06 63.5) (width 0.25) (layer "B.Cu") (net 10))
 (segment (start 99.888 82.992) (end 101.6 81.28) (width 0.6) (layer "B.Cu") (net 10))
 (segment (start 124.46 55.88) (end 116.84 63.5) (width 0.25) (layer "B.Cu") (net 10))
 (segment (start 99.888 97.348) (end 99.888 82.992) (width 0.6) (layer "B.Cu") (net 10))
 (segment (start 72.573 87.813) (end 73.66 88.9) (width 0.25) (layer "B.Cu") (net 10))
 (segment (start 93.98 68.58) (end 73.66 68.58) (width 0.25) (layer "B.Cu") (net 10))
 (segment (start 73.66 68.58) (end 72.573 69.667) (width 0.25) (layer "B.Cu") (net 10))
 (segment (start 99.06 63.5) (end 93.98 68.58) (width 0.25) (layer "B.Cu") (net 10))
 (segment (start 73.66 88.9) (end 72.573 89.987) (width 0.25) (layer "B.Cu") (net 10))
 (segment (start 175.26 58.42) (end 134.62 99.06) (width 0.6) (layer "B.Cu") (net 10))
 (segment (start 96.52 81.28) (end 101.6 86.36) (width 0.25) (layer "F.Cu") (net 2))
 (segment (start 101.6 60.96) (end 96.52 66.04) (width 0.25) (layer "F.Cu") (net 2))
 (segment (start 151.313 54.793) (end 154.94 58.42) (width 0.25) (layer "F.Cu") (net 2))
 (segment (start 114.3 60.96) (end 101.6 60.96) (width 0.25) (layer "F.Cu") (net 2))
 (segment (start 119.38 55.88) (end 114.3 60.96) (width 0.25) (layer "F.Cu") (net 2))
 (segment (start 96.52 66.04) (end 96.52 81.28) (width 0.25) (layer "F.Cu") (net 2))
 (segment (start 120.467 54.793) (end 151.313 54.793) (width 0.25) (layer "F.Cu") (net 2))
 (segment (start 119.38 55.88) (end 120.467 54.793) (width 0.25) (layer "F.Cu") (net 2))
 (segment (start 92.977 54.343) (end 153.403 54.343) (width 0.25) (layer "F.Cu") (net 3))
 (segment (start 73.66 73.66) (end 92.977 54.343) (width 0.25) (layer "F.Cu") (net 3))
 (segment (start 153.403 54.343) (end 157.48 58.42) (width 0.25) (layer "F.Cu") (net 3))
 (segment (start 72.573 73.209749) (end 73.209749 72.573) (width 0.25) (layer "F.Cu") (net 4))
 (segment (start 154.94 53.34) (end 160.02 58.42) (width 0.25) (layer "F.Cu") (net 4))
 (segment (start 72.573 75.113) (end 72.573 73.209749) (width 0.25) (layer "F.Cu") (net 4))
 (segment (start 73.66 76.2) (end 72.573 75.113) (width 0.25) (layer "F.Cu") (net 4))
 (segment (start 93.343251 53.34) (end 154.94 53.34) (width 0.25) (layer "F.Cu") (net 4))
 (segment (start 73.209749 72.573) (end 74.110251 72.573) (width 0.25) (layer "F.Cu") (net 4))
 (segment (start 74.110251 72.573) (end 93.343251 53.34) (width 0.25) (layer "F.Cu") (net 4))
 (segment (start 162.56 58.42) (end 162.56 59.677235) (width 0.25) (layer "F.Cu") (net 5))
 (segment (start 99.51 74.11) (end 101.6 76.2) (width 0.25) (layer "F.Cu") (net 5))
 (segment (start 162.56 59.677235) (end 157.284235 64.953) (width 0.25) (layer "F.Cu") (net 5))
 (segment (start 101.149749 64.953) (end 99.51 66.592749) (width 0.25) (layer "F.Cu") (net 5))
 (segment (start 99.51 66.592749) (end 99.51 74.11) (width 0.25) (layer "F.Cu") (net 5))
 (segment (start 157.284235 64.953) (end 101.149749 64.953) (width 0.25) (layer "F.Cu") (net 5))
 (segment (start 101.149749 87.813) (end 100.513 88.449749) (width 0.25) (layer "B.Cu") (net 6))
 (segment (start 165.1 58.42) (end 152.344 71.176) (width 0.25) (layer "B.Cu") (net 6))
 (segment (start 100.513 88.449749) (end 100.513 92.893) (width 0.25) (layer "B.Cu") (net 6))
 (segment (start 100.513 92.893) (end 101.6 93.98) (width 0.25) (layer "B.Cu") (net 6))
 (segment (start 111.76 83.82) (end 106.043251 83.82) (width 0.25) (layer "B.Cu") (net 6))
 (segment (start 124.404 71.176) (end 111.76 83.82) (width 0.25) (layer "B.Cu") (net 6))
 (segment (start 102.050251 87.813) (end 101.149749 87.813) (width 0.25) (layer "B.Cu") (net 6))
 (segment (start 152.344 71.176) (end 124.404 71.176) (width 0.25) (layer "B.Cu") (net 6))
 (segment (start 106.043251 83.82) (end 102.050251 87.813) (width 0.25) (layer "B.Cu") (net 6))
 (segment (start 167.64 58.396785) (end 133.744 92.292785) (width 0.25) (layer "B.Cu") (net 7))
 (segment (start 133.744 92.292785) (end 133.744 92.952396) (width 0.25) (layer "B.Cu") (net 7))
 (segment (start 128.385396 98.311) (end 103.391 98.311) (width 0.25) (layer "B.Cu") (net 7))
 (segment (start 133.744 92.952396) (end 128.385396 98.311) (width 0.25) (layer "B.Cu") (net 7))
 (segment (start 103.391 98.311) (end 101.6 96.52) (width 0.25) (layer "B.Cu") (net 7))
 (segment (start 132.08 90.17) (end 163.83 90.17) (width 0.6) (layer "F.Cu") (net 8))
 (segment (start 106.68 106.68) (end 116.84 96.52) (width 0.6) (layer "F.Cu") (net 8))
 (segment (start 127 96.52) (end 132.08 91.44) (width 0.6) (layer "F.Cu") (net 8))
 (segment (start 73.66 101.6) (end 78.74 106.68) (width 0.6) (layer "F.Cu") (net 8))
 (segment (start 78.74 106.68) (end 106.68 106.68) (width 0.6) (layer "F.Cu") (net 8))
 (segment (start 132.08 91.44) (end 132.08 90.17) (width 0.6) (layer "F.Cu") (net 8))
 (segment (start 170.18 83.82) (end 170.18 58.42) (width 0.6) (layer "F.Cu") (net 8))
 (segment (start 163.83 90.17) (end 170.18 83.82) (width 0.6) (layer "F.Cu") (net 8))
 (segment (start 116.84 96.52) (end 127 96.52) (width 0.6) (layer "F.Cu") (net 8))
 (segment (start 132.08 85.09) (end 105.41 85.09) (width 0.25) (layer "B.Cu") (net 15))
 (segment (start 105.41 85.09) (end 101.6 88.9) (width 0.25) (layer "B.Cu") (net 15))
 (segment (start 137.16 66.04) (end 101.6 66.04) (width 0.25) (layer "F.Cu") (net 16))
 (segment (start 137.16 78.74) (end 137.16 66.04) (width 0.25) (layer "F.Cu") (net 16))
 (segment (start 132.08 82.55) (end 133.35 82.55) (width 0.25) (layer "F.Cu") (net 16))
 (segment (start 133.35 82.55) (end 137.16 78.74) (width 0.25) (layer "F.Cu") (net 16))
 (segment (start 136.71 66.49) (end 103.69 66.49) (width 0.25) (layer "F.Cu") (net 17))
 (segment (start 103.69 66.49) (end 101.6 68.58) (width 0.25) (layer "F.Cu") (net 17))
 (segment (start 132.08 80.01) (end 136.71 75.38) (width 0.25) (layer "F.Cu") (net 17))
 (segment (start 136.71 75.38) (end 136.71 66.49) (width 0.25) (layer "F.Cu") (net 17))
 (segment (start 134.62 71.12) (end 101.6 71.12) (width 0.25) (layer "F.Cu") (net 18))
 (segment (start 132.08 77.47) (end 134.62 74.93) (width 0.25) (layer "F.Cu") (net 18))
 (segment (start 134.62 74.93) (end 134.62 71.12) (width 0.25) (layer "F.Cu") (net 18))
 (segment (start 103.245 72.015) (end 101.6 73.66) (width 0.25) (layer "F.Cu") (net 19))
 (segment (start 129.165 72.015) (end 103.245 72.015) (width 0.25) (layer "F.Cu") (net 19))
 (segment (start 132.08 74.93) (end 129.165 72.015) (width 0.25) (layer "F.Cu") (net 19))
 (segment (start 133.294 73.604) (end 133.294 92.766) (width 0.25) (layer "B.Cu") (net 20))
 (segment (start 132.08 72.39) (end 133.294 73.604) (width 0.25) (layer "B.Cu") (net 20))
 (segment (start 133.294 92.766) (end 128.199 97.861) (width 0.25) (layer "B.Cu") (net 20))
 (segment (start 128.199 97.861) (end 108.021 97.861) (width 0.25) (layer "B.Cu") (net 20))
 (segment (start 108.021 97.861) (end 101.6 91.44) (width 0.25) (layer "B.Cu") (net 20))
 (segment (start 121.92 55.88) (end 114.3 63.5) (width 0.25) (layer "F.Cu") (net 1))
 (segment (start 101.6 63.5) (end 99.06 66.04) (width 0.25) (layer "F.Cu") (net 1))
 (segment (start 124.46 58.42) (end 152.4 58.42) (width 0.25) (layer "F.Cu") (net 1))
 (segment (start 121.92 55.88) (end 124.46 58.42) (width 0.25) (layer "F.Cu") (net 1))
 (segment (start 99.06 66.04) (end 99.06 81.28) (width 0.25) (layer "F.Cu") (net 1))
 (segment (start 114.3 63.5) (end 101.6 63.5) (width 0.25) (layer "F.Cu") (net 1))
 (segment (start 99.06 81.28) (end 101.6 83.82) (width 0.25) (layer "F.Cu") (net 1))
 (segment (start 101.6 78.74) (end 86.36 78.74) (width 0.6) (layer "B.Cu") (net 9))
 (segment (start 127 55.88) (end 112.48 70.4) (width 0.6) (layer "B.Cu") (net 9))
 (segment (start 170.18 55.88) (end 127 55.88) (width 0.6) (layer "B.Cu") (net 9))
 (segment (start 101.6 101.6) (end 83.82 101.6) (width 0.25) (layer "B.Cu") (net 9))
 (segment (start 83.82 101.6) (end 73.66 91.44) (width 0.25) (layer "B.Cu") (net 9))
 (segment (start 172.72 58.42) (end 170.18 55.88) (width 0.6) (layer "B.Cu") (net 9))
 (segment (start 112.48 70.4) (end 109.94 70.4) (width 0.6) (layer "B.Cu") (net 9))
 (segment (start 86.36 78.74) (end 73.66 91.44) (width 0.6) (layer "B.Cu") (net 9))
 (segment (start 109.94 70.4) (end 101.6 78.74) (width 0.6) (layer "B.Cu") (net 9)))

